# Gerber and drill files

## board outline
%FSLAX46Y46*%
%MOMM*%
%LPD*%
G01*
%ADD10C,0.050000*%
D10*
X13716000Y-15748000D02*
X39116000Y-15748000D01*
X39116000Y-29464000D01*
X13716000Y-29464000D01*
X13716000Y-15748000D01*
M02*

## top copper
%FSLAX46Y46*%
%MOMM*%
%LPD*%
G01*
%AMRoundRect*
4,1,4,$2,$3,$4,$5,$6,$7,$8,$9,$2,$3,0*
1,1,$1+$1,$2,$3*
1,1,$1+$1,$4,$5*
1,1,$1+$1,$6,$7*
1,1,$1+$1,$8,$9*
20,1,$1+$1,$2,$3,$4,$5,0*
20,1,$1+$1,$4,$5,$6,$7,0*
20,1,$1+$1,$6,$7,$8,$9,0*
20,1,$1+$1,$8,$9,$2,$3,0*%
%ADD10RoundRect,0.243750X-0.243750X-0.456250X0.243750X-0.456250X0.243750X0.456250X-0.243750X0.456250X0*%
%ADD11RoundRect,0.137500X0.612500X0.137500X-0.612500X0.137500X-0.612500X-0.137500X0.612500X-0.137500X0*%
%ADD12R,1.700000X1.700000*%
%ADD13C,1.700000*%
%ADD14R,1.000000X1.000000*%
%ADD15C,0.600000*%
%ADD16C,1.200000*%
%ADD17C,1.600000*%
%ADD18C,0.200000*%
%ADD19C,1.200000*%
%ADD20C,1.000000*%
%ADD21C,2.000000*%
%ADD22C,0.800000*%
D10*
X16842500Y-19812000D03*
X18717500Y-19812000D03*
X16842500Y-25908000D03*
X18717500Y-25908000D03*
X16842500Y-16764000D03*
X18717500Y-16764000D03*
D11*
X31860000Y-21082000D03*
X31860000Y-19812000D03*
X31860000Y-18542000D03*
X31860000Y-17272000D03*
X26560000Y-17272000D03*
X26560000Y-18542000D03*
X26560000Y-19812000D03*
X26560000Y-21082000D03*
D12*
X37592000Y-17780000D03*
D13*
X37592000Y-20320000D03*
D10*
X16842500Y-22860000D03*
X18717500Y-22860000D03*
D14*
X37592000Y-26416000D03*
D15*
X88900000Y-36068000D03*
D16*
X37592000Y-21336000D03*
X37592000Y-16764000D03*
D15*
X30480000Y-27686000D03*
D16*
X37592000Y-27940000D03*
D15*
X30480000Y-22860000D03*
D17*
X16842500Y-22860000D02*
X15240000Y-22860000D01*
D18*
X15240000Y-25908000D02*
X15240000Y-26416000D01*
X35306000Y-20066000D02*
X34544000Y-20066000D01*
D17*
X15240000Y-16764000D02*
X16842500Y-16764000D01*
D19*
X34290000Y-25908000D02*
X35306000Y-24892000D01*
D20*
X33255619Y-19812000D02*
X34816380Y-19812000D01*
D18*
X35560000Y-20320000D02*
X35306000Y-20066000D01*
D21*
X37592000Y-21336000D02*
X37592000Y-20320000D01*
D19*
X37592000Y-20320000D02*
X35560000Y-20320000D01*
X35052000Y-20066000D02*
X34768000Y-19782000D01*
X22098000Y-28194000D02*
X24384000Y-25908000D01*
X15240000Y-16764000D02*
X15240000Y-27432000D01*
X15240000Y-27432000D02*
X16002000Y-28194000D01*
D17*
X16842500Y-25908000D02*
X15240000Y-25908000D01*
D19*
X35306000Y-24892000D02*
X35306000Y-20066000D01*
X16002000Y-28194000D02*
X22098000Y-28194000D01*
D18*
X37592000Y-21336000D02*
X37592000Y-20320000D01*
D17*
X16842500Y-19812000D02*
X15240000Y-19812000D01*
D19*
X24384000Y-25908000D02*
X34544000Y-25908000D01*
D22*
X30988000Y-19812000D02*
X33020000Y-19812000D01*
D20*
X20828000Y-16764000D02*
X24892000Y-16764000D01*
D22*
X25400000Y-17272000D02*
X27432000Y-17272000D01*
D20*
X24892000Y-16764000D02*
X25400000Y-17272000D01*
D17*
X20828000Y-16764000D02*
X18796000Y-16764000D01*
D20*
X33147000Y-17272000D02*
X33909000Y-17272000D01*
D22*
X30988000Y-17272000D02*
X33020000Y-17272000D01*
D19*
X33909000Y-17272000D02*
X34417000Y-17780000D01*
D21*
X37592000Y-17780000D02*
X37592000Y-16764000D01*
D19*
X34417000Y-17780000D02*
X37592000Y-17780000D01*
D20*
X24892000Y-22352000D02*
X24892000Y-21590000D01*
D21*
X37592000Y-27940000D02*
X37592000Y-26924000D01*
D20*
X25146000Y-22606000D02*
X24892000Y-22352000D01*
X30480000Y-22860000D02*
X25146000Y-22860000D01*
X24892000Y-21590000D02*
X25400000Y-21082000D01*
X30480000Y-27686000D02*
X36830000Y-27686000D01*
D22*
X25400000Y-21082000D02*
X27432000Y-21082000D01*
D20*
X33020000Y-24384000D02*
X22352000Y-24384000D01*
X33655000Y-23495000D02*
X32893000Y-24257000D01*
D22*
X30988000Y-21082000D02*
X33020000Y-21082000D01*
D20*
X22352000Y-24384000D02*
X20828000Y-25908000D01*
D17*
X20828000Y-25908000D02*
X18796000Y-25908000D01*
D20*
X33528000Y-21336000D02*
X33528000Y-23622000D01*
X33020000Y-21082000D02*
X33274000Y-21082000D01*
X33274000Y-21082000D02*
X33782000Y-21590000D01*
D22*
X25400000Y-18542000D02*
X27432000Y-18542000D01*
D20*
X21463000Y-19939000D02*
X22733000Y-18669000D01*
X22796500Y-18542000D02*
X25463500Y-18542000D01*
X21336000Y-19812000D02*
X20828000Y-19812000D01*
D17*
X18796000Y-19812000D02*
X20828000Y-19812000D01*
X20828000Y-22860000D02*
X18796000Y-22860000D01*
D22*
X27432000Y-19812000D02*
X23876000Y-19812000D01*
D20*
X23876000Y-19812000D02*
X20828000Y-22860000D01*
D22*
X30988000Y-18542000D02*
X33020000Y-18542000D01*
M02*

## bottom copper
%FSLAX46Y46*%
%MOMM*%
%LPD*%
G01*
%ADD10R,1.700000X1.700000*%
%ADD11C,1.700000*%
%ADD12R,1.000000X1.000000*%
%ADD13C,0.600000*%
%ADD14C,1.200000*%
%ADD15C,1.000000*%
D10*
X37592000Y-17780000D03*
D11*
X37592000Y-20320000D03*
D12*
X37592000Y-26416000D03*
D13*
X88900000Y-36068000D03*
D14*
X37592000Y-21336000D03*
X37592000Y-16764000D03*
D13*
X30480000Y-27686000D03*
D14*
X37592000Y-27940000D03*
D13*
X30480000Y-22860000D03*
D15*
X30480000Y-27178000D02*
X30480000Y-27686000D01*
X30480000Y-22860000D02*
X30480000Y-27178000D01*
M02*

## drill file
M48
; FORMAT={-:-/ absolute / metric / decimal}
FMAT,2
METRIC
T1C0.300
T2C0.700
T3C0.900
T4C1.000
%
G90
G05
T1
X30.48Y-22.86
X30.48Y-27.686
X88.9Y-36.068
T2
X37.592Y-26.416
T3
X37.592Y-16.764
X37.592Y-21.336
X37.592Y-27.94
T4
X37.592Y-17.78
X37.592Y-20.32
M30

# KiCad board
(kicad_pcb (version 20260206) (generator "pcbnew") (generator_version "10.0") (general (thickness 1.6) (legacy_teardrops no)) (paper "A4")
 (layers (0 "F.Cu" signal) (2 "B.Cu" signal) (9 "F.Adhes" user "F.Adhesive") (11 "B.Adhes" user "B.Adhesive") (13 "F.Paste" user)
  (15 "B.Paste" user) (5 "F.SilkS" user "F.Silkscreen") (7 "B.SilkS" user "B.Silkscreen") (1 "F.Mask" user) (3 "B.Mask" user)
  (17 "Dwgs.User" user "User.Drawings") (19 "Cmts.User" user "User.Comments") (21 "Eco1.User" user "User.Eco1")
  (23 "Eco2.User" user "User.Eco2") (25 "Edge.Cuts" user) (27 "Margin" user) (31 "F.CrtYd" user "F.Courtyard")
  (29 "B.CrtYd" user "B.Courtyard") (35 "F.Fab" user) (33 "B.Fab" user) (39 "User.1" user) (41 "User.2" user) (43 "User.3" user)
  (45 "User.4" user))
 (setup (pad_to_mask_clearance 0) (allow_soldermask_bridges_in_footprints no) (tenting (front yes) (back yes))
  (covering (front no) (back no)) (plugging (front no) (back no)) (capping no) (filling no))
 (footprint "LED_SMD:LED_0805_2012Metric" (layer "F.Cu") (at 17.78 19.812)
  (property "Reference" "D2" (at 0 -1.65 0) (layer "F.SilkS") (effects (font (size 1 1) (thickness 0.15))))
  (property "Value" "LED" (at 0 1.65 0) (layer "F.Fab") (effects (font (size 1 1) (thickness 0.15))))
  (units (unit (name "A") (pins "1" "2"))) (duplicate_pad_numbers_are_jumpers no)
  (pad "1" smd roundrect (at -0.9375 0) (size 0.975 1.4) (layers "F.Cu" "F.Mask" "F.Paste") (roundrect_rratio 0.25) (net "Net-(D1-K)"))
  (pad "2" smd roundrect (at 0.9375 0) (size 0.975 1.4) (layers "F.Cu" "F.Mask" "F.Paste") (roundrect_rratio 0.25) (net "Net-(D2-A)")))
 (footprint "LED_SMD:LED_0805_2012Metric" (layer "F.Cu") (at 17.78 25.908)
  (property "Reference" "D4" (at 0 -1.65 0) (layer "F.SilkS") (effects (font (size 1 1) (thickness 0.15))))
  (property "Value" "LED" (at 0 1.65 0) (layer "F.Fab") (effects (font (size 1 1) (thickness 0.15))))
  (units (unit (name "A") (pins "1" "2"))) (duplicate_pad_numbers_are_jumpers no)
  (pad "1" smd roundrect (at -0.9375 0) (size 0.975 1.4) (layers "F.Cu" "F.Mask" "F.Paste") (roundrect_rratio 0.25) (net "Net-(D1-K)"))
  (pad "2" smd roundrect (at 0.9375 0) (size 0.975 1.4) (layers "F.Cu" "F.Mask" "F.Paste") (roundrect_rratio 0.25) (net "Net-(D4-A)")))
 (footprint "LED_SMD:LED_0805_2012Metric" (layer "F.Cu") (at 17.78 16.764)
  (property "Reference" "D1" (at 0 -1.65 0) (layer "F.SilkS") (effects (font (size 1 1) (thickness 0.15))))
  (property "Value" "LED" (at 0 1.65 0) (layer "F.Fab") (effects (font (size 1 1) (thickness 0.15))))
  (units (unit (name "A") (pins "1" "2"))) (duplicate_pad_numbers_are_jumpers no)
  (pad "1" smd roundrect (at -0.9375 0) (size 0.975 1.4) (layers "F.Cu" "F.Mask" "F.Paste") (roundrect_rratio 0.25) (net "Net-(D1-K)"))
  (pad "2" smd roundrect (at 0.9375 0) (size 0.975 1.4) (layers "F.Cu" "F.Mask" "F.Paste") (roundrect_rratio 0.25) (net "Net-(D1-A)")))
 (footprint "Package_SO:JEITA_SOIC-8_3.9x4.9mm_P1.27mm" (layer "F.Cu") (at 29.21 19.177 180)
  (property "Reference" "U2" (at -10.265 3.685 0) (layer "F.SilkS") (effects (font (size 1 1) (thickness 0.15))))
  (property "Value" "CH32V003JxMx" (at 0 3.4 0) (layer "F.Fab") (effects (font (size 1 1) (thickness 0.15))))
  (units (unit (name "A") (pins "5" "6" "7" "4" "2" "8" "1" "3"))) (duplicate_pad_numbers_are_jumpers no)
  (pad "1" smd roundrect (at -2.65 -1.905 180) (size 1.5 0.55) (layers "F.Cu" "F.Mask" "F.Paste") (roundrect_rratio 0.25) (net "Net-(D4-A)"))
  (pad "2" smd roundrect (at -2.65 -0.635 180) (size 1.5 0.55) (layers "F.Cu" "F.Mask" "F.Paste") (roundrect_rratio 0.25) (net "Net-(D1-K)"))
  (pad "3" smd roundrect (at -2.65 0.635 180) (size 1.5 0.55) (layers "F.Cu" "F.Mask" "F.Paste") (roundrect_rratio 0.25)
   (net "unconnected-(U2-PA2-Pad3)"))
  (pad "4" smd roundrect (at -2.65 1.905 180) (size 1.5 0.55) (layers "F.Cu" "F.Mask" "F.Paste") (roundrect_rratio 0.25)
   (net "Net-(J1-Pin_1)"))
  (pad "5" smd roundrect (at 2.65 1.905 180) (size 1.5 0.55) (layers "F.Cu" "F.Mask" "F.Paste") (roundrect_rratio 0.25) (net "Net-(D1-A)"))
  (pad "6" smd roundrect (at 2.65 0.635 180) (size 1.5 0.55) (layers "F.Cu" "F.Mask" "F.Paste") (roundrect_rratio 0.25) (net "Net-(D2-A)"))
  (pad "7" smd roundrect (at 2.65 -0.635 180) (size 1.5 0.55) (layers "F.Cu" "F.Mask" "F.Paste") (roundrect_rratio 0.25) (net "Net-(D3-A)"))
  (pad "8" smd roundrect (at 2.65 -1.905 180) (size 1.5 0.55) (layers "F.Cu" "F.Mask" "F.Paste") (roundrect_rratio 0.25)
   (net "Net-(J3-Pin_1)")))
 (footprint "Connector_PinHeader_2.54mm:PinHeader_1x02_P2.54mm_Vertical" (layer "F.Cu") (at 37.592 17.78)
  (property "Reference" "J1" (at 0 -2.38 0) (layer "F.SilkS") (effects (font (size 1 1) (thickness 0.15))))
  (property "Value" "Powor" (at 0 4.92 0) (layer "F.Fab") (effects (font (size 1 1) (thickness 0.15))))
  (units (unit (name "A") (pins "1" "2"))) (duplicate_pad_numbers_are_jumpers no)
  (pad "1" thru_hole rect (at 0 0) (size 1.7 1.7) (drill 1) (layers "*.Cu" "*.Mask") (remove_unused_layers no) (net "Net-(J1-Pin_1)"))
  (pad "2" thru_hole circle (at 0 2.54) (size 1.7 1.7) (drill 1) (layers "*.Cu" "*.Mask") (remove_unused_layers no) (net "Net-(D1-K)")))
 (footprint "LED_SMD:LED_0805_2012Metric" (layer "F.Cu") (at 17.78 22.86)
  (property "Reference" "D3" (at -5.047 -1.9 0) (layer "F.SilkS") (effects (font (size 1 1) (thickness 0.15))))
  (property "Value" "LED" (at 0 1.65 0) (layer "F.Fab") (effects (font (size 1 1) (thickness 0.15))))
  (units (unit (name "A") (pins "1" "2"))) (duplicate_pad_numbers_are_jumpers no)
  (pad "1" smd roundrect (at -0.9375 0) (size 0.975 1.4) (layers "F.Cu" "F.Mask" "F.Paste") (roundrect_rratio 0.25) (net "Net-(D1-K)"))
  (pad "2" smd roundrect (at 0.9375 0) (size 0.975 1.4) (layers "F.Cu" "F.Mask" "F.Paste") (roundrect_rratio 0.25) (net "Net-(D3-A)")))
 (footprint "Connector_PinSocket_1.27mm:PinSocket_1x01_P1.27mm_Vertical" (layer "F.Cu") (at 37.592 26.416)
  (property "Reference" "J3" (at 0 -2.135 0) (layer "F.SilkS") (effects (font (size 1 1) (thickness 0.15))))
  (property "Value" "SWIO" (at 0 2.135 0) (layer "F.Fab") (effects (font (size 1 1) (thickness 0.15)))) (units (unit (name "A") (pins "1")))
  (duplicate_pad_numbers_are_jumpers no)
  (pad "1" thru_hole rect (at 0 0) (size 1 1) (drill 0.7) (layers "*.Cu" "*.Mask") (remove_unused_layers no) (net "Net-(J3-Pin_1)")))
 (gr_rect (start 13.716 15.748) (end 39.116 29.464) (stroke (width 0.05) (type default)) (fill no) (layer "Edge.Cuts"))
 (via (at 88.9 36.068) (size 0.6) (drill 0.3) (layers "F.Cu" "B.Cu") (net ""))
 (segment (start 16.8425 22.86) (end 15.24 22.86) (width 1.6) (layer "F.Cu") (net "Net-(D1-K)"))
 (segment (start 15.24 25.908) (end 15.24 26.416) (width 0.2) (layer "F.Cu") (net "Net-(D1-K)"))
 (segment (start 35.306 20.066) (end 34.544 20.066) (width 0.2) (layer "F.Cu") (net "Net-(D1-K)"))
 (segment (start 15.24 16.764) (end 16.8425 16.764) (width 1.6) (layer "F.Cu") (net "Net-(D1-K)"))
 (segment (start 34.29 25.908) (end 35.306 24.892) (width 1.2) (layer "F.Cu") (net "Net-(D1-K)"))
 (segment (start 33.255619 19.812) (end 34.81638 19.812) (width 1) (layer "F.Cu") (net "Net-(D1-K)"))
 (segment (start 35.56 20.32) (end 35.306 20.066) (width 0.2) (layer "F.Cu") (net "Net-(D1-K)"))
 (segment (start 37.592 21.336) (end 37.592 20.32) (width 2) (layer "F.Cu") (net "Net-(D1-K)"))
 (segment (start 37.592 20.32) (end 35.56 20.32) (width 1.2) (layer "F.Cu") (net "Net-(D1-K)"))
 (segment (start 35.052 20.066) (end 34.768 19.782) (width 1.2) (layer "F.Cu") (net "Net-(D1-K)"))
 (segment (start 22.098 28.194) (end 24.384 25.908) (width 1.2) (layer "F.Cu") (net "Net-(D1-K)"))
 (segment (start 15.24 16.764) (end 15.24 27.432) (width 1.2) (layer "F.Cu") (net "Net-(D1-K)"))
 (segment (start 15.24 27.432) (end 16.002 28.194) (width 1.2) (layer "F.Cu") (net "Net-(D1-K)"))
 (segment (start 16.8425 25.908) (end 15.24 25.908) (width 1.6) (layer "F.Cu") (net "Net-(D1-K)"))
 (segment (start 35.306 24.892) (end 35.306 20.066) (width 1.2) (layer "F.Cu") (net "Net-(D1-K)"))
 (segment (start 16.002 28.194) (end 22.098 28.194) (width 1.2) (layer "F.Cu") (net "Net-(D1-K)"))
 (segment (start 37.592 21.336) (end 37.592 20.32) (width 0.2) (layer "F.Cu") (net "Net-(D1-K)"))
 (segment (start 16.8425 19.812) (end 15.24 19.812) (width 1.6) (layer "F.Cu") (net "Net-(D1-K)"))
 (segment (start 24.384 25.908) (end 34.544 25.908) (width 1.2) (layer "F.Cu") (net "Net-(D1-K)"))
 (segment (start 30.988 19.812) (end 33.02 19.812) (width 0.8) (layer "F.Cu") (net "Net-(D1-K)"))
 (via (at 37.592 21.336) (size 1.2) (drill 0.9) (layers "F.Cu" "B.Cu") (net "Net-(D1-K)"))
 (segment (start 20.828 16.764) (end 24.892 16.764) (width 1) (layer "F.Cu") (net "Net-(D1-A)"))
 (segment (start 25.4 17.272) (end 27.432 17.272) (width 0.8) (layer "F.Cu") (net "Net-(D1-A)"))
 (segment (start 24.892 16.764) (end 25.4 17.272) (width 1) (layer "F.Cu") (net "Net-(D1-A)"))
 (segment (start 20.828 16.764) (end 18.796 16.764) (width 1.6) (layer "F.Cu") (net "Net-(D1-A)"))
 (segment (start 33.147 17.272) (end 33.909 17.272) (width 1) (layer "F.Cu") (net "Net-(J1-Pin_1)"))
 (segment (start 30.988 17.272) (end 33.02 17.272) (width 0.8) (layer "F.Cu") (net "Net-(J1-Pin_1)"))
 (segment (start 33.909 17.272) (end 34.417 17.78) (width 1.2) (layer "F.Cu") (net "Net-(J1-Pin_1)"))
 (segment (start 37.592 17.78) (end 37.592 16.764) (width 2) (layer "F.Cu") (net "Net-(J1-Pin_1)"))
 (segment (start 34.417 17.78) (end 37.592 17.78) (width 1.2) (layer "F.Cu") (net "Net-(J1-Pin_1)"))
 (via (at 37.592 16.764) (size 1.2) (drill 0.9) (layers "F.Cu" "B.Cu") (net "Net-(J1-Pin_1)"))
 (segment (start 24.892 22.352) (end 24.892 21.59) (width 1) (layer "F.Cu") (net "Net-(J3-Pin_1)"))
 (segment (start 37.592 27.94) (end 37.592 26.924) (width 2) (layer "F.Cu") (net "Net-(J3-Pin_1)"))
 (segment (start 25.146 22.606) (end 24.892 22.352) (width 1) (layer "F.Cu") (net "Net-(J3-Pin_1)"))
 (segment (start 30.48 22.86) (end 25.146 22.86) (width 1) (layer "F.Cu") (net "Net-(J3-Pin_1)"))
 (segment (start 24.892 21.59) (end 25.4 21.082) (width 1) (layer "F.Cu") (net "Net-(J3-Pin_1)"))
 (segment (start 30.48 27.686) (end 36.83 27.686) (width 1) (layer "F.Cu") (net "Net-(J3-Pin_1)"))
 (segment (start 25.4 21.082) (end 27.432 21.082) (width 0.8) (layer "F.Cu") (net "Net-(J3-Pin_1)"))
 (via (at 30.48 27.686) (size 0.6) (drill 0.3) (layers "F.Cu" "B.Cu") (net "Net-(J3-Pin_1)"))
 (via (at 37.592 27.94) (size 1.2) (drill 0.9) (layers "F.Cu" "B.Cu") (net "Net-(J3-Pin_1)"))
 (via (at 30.48 22.86) (size 0.6) (drill 0.3) (layers "F.Cu" "B.Cu") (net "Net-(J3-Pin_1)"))
 (segment (start 30.48 27.178) (end 30.48 27.686) (width 1) (layer "B.Cu") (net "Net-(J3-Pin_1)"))
 (segment (start 30.48 22.86) (end 30.48 27.178) (width 1) (layer "B.Cu") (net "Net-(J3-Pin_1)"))
 (segment (start 33.02 24.384) (end 22.352 24.384) (width 1) (layer "F.Cu") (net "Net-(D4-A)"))
 (segment (start 33.655 23.495) (end 32.893 24.257) (width 1) (layer "F.Cu") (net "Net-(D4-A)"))
 (segment (start 30.988 21.082) (end 33.02 21.082) (width 0.8) (layer "F.Cu") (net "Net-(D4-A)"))
 (segment (start 22.352 24.384) (end 20.828 25.908) (width 1) (layer "F.Cu") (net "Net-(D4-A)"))
 (segment (start 20.828 25.908) (end 18.796 25.908) (width 1.6) (layer "F.Cu") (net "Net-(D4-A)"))
 (segment (start 33.528 21.336) (end 33.528 23.622) (width 1) (layer "F.Cu") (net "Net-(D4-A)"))
 (segment (start 33.02 21.082) (end 33.274 21.082) (width 1) (layer "F.Cu") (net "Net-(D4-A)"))
 (segment (start 33.274 21.082) (end 33.782 21.59) (width 1) (layer "F.Cu") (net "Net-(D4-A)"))
 (segment (start 25.4 18.542) (end 27.432 18.542) (width 0.8) (layer "F.Cu") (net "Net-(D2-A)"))
 (segment (start 21.463 19.939) (end 22.733 18.669) (width 1) (layer "F.Cu") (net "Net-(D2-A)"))
 (segment (start 22.7965 18.542) (end 25.4635 18.542) (width 1) (layer "F.Cu") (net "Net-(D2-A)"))
 (segment (start 21.336 19.812) (end 20.828 19.812) (width 1) (layer "F.Cu") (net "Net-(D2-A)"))
 (segment (start 18.796 19.812) (end 20.828 19.812) (width 1.6) (layer "F.Cu") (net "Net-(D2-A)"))
 (segment (start 20.828 22.86) (end 18.796 22.86) (width 1.6) (layer "F.Cu") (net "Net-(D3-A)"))
 (segment (start 27.432 19.812) (end 23.876 19.812) (width 0.8) (layer "F.Cu") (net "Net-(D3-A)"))
 (segment (start 23.876 19.812) (end 20.828 22.86) (width 1) (layer "F.Cu") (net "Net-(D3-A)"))
 (segment (start 30.988 18.542) (end 33.02 18.542) (width 0.8) (layer "F.Cu") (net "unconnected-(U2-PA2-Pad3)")))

